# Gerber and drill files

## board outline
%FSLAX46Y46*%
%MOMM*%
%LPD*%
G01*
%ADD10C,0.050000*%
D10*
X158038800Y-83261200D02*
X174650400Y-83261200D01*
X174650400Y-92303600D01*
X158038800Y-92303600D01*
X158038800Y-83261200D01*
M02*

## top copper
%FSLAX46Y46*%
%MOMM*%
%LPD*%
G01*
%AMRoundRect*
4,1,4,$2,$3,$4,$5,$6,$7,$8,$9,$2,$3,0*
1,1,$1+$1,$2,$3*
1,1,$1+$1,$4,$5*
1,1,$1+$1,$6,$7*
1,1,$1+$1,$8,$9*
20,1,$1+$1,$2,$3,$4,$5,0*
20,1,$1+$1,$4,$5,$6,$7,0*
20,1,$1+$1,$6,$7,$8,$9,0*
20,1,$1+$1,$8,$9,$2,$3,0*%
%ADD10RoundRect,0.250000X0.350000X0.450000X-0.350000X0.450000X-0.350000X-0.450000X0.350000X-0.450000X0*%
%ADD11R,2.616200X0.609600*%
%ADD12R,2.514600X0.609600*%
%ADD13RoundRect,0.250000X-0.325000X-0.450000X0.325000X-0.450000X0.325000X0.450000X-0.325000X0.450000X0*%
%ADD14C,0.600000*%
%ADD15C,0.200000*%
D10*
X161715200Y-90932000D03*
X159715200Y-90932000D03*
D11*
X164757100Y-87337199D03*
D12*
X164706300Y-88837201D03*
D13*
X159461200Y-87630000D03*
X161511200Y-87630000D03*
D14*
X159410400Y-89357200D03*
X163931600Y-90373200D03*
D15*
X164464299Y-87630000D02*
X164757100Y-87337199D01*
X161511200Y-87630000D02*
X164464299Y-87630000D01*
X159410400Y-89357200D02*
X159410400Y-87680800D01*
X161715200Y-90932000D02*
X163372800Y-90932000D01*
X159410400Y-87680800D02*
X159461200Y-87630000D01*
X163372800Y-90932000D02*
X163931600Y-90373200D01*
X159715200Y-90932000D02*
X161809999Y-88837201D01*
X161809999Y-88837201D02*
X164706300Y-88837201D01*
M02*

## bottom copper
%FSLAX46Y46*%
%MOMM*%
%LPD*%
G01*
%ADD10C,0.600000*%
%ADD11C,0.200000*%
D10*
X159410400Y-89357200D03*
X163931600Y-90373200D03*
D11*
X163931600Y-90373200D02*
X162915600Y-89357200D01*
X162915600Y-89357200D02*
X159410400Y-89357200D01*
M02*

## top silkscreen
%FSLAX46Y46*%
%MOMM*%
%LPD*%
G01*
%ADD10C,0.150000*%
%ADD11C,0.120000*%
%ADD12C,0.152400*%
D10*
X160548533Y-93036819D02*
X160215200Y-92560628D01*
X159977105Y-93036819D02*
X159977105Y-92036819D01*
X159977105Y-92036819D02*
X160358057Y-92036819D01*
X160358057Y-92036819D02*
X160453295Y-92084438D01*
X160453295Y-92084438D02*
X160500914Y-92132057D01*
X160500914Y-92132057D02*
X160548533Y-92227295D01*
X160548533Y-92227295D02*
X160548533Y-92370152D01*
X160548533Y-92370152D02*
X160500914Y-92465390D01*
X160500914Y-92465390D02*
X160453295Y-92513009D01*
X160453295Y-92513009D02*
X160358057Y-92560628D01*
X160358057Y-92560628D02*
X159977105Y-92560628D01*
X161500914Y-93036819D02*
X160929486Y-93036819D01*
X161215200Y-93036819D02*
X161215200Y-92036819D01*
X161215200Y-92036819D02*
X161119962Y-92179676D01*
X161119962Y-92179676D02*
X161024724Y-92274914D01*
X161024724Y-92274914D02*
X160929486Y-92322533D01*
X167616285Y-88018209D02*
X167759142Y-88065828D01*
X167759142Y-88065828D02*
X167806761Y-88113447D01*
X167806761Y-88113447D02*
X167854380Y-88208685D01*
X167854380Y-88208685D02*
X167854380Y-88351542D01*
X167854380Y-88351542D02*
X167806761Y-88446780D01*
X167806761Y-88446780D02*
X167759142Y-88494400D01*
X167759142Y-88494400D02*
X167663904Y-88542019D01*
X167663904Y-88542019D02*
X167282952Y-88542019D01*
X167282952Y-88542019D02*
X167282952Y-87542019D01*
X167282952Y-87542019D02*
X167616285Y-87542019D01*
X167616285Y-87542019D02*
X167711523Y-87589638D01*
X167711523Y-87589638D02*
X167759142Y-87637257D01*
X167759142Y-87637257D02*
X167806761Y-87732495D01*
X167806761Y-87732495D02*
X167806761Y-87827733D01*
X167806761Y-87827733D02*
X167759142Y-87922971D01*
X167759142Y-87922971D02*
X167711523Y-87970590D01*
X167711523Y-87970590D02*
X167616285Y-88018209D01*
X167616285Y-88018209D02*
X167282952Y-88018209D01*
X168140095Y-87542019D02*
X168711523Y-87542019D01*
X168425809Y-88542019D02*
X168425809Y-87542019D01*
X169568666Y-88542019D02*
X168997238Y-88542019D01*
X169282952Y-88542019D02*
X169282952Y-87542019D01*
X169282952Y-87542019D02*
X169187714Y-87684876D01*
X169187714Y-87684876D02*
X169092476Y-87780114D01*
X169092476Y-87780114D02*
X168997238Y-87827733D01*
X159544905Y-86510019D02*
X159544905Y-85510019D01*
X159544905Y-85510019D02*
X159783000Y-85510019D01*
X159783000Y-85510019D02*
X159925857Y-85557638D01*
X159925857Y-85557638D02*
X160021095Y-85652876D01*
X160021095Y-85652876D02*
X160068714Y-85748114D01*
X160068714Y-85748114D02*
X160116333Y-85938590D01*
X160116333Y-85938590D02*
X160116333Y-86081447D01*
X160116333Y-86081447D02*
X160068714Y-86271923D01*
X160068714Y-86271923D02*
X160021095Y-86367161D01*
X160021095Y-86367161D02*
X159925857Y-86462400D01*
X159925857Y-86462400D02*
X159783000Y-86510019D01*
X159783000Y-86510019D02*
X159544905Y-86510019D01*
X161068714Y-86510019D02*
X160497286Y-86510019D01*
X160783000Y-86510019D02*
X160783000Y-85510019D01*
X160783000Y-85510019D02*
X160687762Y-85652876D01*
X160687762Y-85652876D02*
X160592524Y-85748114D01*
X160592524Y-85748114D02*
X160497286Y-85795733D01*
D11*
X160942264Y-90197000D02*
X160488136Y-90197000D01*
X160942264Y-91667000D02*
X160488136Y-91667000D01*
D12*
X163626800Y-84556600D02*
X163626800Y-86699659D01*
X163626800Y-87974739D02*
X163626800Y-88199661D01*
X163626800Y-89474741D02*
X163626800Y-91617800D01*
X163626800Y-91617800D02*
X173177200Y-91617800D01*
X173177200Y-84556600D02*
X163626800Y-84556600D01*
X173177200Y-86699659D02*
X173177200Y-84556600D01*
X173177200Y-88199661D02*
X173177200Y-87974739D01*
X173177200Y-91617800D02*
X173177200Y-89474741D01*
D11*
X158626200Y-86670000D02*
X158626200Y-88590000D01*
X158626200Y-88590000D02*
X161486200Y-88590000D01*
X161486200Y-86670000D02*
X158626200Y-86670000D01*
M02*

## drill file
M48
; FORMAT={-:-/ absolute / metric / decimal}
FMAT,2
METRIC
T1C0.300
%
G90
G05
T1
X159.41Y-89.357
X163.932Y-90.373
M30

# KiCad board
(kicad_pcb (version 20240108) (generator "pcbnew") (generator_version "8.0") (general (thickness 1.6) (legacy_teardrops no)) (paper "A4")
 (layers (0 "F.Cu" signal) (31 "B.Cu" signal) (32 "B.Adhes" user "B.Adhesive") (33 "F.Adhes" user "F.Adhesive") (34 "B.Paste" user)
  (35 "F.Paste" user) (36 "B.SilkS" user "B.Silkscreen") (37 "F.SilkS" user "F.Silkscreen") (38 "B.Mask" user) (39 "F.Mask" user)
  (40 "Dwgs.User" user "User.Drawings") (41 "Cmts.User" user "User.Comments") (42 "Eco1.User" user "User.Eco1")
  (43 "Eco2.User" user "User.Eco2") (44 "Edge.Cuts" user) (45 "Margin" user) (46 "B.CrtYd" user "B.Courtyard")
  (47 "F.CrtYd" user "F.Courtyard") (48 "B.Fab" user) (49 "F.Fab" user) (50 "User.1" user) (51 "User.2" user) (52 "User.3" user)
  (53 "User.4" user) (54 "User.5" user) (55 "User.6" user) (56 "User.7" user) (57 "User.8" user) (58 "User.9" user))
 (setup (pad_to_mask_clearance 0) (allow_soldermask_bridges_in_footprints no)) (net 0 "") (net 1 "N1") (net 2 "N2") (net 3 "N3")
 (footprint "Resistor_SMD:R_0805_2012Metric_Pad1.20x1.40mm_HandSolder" (layer "F.Cu") (at 160.7152 90.932 180)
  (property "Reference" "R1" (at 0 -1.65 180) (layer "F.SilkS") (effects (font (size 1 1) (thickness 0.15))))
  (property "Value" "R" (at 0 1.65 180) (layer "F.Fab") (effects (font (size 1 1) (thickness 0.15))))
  (fp_line (start -0.227064 0.735) (end 0.227064 0.735) (stroke (width 0.12) (type solid)) (layer "F.SilkS"))
  (fp_line (start -0.227064 -0.735) (end 0.227064 -0.735) (stroke (width 0.12) (type solid)) (layer "F.SilkS"))
  (pad "1" smd roundrect (at -1 0 180) (size 1.2 1.4) (layers "F.Cu" "F.Paste" "F.Mask") (roundrect_rratio 0.208333) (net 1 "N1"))
  (pad "2" smd roundrect (at 1 0 180) (size 1.2 1.4) (layers "F.Cu" "F.Paste" "F.Mask") (roundrect_rratio 0.208333) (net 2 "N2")))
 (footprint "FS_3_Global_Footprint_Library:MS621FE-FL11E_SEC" (layer "F.Cu") (at 168.402 88.0872)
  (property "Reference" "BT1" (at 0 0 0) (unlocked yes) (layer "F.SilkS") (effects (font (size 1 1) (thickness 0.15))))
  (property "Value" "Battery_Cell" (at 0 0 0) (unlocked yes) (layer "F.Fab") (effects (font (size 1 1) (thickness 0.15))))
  (fp_line (start -4.7752 -3.5306) (end -4.7752 -1.387541) (stroke (width 0.1524) (type solid)) (layer "F.SilkS"))
  (fp_line (start -4.7752 -0.112461) (end -4.7752 0.112461) (stroke (width 0.1524) (type solid)) (layer "F.SilkS"))
  (fp_line (start -4.7752 1.387541) (end -4.7752 3.5306) (stroke (width 0.1524) (type solid)) (layer "F.SilkS"))
  (fp_line (start -4.7752 3.5306) (end 4.7752 3.5306) (stroke (width 0.1524) (type solid)) (layer "F.SilkS"))
  (fp_line (start 4.7752 -3.5306) (end -4.7752 -3.5306) (stroke (width 0.1524) (type solid)) (layer "F.SilkS"))
  (fp_line (start 4.7752 -1.387541) (end 4.7752 -3.5306) (stroke (width 0.1524) (type solid)) (layer "F.SilkS"))
  (fp_line (start 4.7752 0.112461) (end 4.7752 -0.112461) (stroke (width 0.1524) (type solid)) (layer "F.SilkS"))
  (fp_line (start 4.7752 3.5306) (end 4.7752 1.387541) (stroke (width 0.1524) (type solid)) (layer "F.SilkS"))
  (pad "1" smd rect (at -3.6449 -0.750001) (size 2.6162 0.6096) (layers "F.Cu" "F.Paste" "F.Mask") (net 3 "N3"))
  (pad "2" smd rect (at -3.6957 0.750001) (size 2.5146 0.6096) (layers "F.Cu" "F.Paste" "F.Mask") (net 2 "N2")))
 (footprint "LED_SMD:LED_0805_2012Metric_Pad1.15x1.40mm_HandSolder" (layer "F.Cu") (at 160.4862 87.63)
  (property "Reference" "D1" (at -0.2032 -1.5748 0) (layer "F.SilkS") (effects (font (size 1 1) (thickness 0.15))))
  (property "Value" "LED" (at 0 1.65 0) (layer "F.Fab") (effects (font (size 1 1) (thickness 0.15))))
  (fp_line (start -1.86 -0.96) (end -1.86 0.96) (stroke (width 0.12) (type solid)) (layer "F.SilkS"))
  (fp_line (start -1.86 0.96) (end 1 0.96) (stroke (width 0.12) (type solid)) (layer "F.SilkS"))
  (fp_line (start 1 -0.96) (end -1.86 -0.96) (stroke (width 0.12) (type solid)) (layer "F.SilkS"))
  (pad "1" smd roundrect (at -1.025 0) (size 1.15 1.4) (layers "F.Cu" "F.Paste" "F.Mask") (roundrect_rratio 0.217391) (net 1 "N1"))
  (pad "2" smd roundrect (at 1.025 0) (size 1.15 1.4) (layers "F.Cu" "F.Paste" "F.Mask") (roundrect_rratio 0.217391) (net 3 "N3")))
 (gr_rect (start 158.0388 83.2612) (end 174.6504 92.3036) (stroke (width 0.05) (type default)) (fill none) (layer "Edge.Cuts"))
 (segment (start 164.464299 87.63) (end 164.7571 87.337199) (width 0.2) (layer "F.Cu") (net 3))
 (segment (start 161.5112 87.63) (end 164.464299 87.63) (width 0.2) (layer "F.Cu") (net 3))
 (segment (start 159.4104 89.3572) (end 159.4104 87.6808) (width 0.2) (layer "F.Cu") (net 1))
 (segment (start 161.7152 90.932) (end 163.3728 90.932) (width 0.2) (layer "F.Cu") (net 1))
 (segment (start 159.4104 87.6808) (end 159.4612 87.63) (width 0.2) (layer "F.Cu") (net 1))
 (segment (start 163.3728 90.932) (end 163.9316 90.3732) (width 0.2) (layer "F.Cu") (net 1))
 (via (at 159.4104 89.3572) (size 0.6) (drill 0.3) (layers "F.Cu" "B.Cu") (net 1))
 (via (at 163.9316 90.3732) (size 0.6) (drill 0.3) (layers "F.Cu" "B.Cu") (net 1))
 (segment (start 163.9316 90.3732) (end 162.9156 89.3572) (width 0.2) (layer "B.Cu") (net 1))
 (segment (start 162.9156 89.3572) (end 159.4104 89.3572) (width 0.2) (layer "B.Cu") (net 1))
 (segment (start 159.7152 90.932) (end 161.809999 88.837201) (width 0.2) (layer "F.Cu") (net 2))
 (segment (start 161.809999 88.837201) (end 164.7063 88.837201) (width 0.2) (layer "F.Cu") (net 2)))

